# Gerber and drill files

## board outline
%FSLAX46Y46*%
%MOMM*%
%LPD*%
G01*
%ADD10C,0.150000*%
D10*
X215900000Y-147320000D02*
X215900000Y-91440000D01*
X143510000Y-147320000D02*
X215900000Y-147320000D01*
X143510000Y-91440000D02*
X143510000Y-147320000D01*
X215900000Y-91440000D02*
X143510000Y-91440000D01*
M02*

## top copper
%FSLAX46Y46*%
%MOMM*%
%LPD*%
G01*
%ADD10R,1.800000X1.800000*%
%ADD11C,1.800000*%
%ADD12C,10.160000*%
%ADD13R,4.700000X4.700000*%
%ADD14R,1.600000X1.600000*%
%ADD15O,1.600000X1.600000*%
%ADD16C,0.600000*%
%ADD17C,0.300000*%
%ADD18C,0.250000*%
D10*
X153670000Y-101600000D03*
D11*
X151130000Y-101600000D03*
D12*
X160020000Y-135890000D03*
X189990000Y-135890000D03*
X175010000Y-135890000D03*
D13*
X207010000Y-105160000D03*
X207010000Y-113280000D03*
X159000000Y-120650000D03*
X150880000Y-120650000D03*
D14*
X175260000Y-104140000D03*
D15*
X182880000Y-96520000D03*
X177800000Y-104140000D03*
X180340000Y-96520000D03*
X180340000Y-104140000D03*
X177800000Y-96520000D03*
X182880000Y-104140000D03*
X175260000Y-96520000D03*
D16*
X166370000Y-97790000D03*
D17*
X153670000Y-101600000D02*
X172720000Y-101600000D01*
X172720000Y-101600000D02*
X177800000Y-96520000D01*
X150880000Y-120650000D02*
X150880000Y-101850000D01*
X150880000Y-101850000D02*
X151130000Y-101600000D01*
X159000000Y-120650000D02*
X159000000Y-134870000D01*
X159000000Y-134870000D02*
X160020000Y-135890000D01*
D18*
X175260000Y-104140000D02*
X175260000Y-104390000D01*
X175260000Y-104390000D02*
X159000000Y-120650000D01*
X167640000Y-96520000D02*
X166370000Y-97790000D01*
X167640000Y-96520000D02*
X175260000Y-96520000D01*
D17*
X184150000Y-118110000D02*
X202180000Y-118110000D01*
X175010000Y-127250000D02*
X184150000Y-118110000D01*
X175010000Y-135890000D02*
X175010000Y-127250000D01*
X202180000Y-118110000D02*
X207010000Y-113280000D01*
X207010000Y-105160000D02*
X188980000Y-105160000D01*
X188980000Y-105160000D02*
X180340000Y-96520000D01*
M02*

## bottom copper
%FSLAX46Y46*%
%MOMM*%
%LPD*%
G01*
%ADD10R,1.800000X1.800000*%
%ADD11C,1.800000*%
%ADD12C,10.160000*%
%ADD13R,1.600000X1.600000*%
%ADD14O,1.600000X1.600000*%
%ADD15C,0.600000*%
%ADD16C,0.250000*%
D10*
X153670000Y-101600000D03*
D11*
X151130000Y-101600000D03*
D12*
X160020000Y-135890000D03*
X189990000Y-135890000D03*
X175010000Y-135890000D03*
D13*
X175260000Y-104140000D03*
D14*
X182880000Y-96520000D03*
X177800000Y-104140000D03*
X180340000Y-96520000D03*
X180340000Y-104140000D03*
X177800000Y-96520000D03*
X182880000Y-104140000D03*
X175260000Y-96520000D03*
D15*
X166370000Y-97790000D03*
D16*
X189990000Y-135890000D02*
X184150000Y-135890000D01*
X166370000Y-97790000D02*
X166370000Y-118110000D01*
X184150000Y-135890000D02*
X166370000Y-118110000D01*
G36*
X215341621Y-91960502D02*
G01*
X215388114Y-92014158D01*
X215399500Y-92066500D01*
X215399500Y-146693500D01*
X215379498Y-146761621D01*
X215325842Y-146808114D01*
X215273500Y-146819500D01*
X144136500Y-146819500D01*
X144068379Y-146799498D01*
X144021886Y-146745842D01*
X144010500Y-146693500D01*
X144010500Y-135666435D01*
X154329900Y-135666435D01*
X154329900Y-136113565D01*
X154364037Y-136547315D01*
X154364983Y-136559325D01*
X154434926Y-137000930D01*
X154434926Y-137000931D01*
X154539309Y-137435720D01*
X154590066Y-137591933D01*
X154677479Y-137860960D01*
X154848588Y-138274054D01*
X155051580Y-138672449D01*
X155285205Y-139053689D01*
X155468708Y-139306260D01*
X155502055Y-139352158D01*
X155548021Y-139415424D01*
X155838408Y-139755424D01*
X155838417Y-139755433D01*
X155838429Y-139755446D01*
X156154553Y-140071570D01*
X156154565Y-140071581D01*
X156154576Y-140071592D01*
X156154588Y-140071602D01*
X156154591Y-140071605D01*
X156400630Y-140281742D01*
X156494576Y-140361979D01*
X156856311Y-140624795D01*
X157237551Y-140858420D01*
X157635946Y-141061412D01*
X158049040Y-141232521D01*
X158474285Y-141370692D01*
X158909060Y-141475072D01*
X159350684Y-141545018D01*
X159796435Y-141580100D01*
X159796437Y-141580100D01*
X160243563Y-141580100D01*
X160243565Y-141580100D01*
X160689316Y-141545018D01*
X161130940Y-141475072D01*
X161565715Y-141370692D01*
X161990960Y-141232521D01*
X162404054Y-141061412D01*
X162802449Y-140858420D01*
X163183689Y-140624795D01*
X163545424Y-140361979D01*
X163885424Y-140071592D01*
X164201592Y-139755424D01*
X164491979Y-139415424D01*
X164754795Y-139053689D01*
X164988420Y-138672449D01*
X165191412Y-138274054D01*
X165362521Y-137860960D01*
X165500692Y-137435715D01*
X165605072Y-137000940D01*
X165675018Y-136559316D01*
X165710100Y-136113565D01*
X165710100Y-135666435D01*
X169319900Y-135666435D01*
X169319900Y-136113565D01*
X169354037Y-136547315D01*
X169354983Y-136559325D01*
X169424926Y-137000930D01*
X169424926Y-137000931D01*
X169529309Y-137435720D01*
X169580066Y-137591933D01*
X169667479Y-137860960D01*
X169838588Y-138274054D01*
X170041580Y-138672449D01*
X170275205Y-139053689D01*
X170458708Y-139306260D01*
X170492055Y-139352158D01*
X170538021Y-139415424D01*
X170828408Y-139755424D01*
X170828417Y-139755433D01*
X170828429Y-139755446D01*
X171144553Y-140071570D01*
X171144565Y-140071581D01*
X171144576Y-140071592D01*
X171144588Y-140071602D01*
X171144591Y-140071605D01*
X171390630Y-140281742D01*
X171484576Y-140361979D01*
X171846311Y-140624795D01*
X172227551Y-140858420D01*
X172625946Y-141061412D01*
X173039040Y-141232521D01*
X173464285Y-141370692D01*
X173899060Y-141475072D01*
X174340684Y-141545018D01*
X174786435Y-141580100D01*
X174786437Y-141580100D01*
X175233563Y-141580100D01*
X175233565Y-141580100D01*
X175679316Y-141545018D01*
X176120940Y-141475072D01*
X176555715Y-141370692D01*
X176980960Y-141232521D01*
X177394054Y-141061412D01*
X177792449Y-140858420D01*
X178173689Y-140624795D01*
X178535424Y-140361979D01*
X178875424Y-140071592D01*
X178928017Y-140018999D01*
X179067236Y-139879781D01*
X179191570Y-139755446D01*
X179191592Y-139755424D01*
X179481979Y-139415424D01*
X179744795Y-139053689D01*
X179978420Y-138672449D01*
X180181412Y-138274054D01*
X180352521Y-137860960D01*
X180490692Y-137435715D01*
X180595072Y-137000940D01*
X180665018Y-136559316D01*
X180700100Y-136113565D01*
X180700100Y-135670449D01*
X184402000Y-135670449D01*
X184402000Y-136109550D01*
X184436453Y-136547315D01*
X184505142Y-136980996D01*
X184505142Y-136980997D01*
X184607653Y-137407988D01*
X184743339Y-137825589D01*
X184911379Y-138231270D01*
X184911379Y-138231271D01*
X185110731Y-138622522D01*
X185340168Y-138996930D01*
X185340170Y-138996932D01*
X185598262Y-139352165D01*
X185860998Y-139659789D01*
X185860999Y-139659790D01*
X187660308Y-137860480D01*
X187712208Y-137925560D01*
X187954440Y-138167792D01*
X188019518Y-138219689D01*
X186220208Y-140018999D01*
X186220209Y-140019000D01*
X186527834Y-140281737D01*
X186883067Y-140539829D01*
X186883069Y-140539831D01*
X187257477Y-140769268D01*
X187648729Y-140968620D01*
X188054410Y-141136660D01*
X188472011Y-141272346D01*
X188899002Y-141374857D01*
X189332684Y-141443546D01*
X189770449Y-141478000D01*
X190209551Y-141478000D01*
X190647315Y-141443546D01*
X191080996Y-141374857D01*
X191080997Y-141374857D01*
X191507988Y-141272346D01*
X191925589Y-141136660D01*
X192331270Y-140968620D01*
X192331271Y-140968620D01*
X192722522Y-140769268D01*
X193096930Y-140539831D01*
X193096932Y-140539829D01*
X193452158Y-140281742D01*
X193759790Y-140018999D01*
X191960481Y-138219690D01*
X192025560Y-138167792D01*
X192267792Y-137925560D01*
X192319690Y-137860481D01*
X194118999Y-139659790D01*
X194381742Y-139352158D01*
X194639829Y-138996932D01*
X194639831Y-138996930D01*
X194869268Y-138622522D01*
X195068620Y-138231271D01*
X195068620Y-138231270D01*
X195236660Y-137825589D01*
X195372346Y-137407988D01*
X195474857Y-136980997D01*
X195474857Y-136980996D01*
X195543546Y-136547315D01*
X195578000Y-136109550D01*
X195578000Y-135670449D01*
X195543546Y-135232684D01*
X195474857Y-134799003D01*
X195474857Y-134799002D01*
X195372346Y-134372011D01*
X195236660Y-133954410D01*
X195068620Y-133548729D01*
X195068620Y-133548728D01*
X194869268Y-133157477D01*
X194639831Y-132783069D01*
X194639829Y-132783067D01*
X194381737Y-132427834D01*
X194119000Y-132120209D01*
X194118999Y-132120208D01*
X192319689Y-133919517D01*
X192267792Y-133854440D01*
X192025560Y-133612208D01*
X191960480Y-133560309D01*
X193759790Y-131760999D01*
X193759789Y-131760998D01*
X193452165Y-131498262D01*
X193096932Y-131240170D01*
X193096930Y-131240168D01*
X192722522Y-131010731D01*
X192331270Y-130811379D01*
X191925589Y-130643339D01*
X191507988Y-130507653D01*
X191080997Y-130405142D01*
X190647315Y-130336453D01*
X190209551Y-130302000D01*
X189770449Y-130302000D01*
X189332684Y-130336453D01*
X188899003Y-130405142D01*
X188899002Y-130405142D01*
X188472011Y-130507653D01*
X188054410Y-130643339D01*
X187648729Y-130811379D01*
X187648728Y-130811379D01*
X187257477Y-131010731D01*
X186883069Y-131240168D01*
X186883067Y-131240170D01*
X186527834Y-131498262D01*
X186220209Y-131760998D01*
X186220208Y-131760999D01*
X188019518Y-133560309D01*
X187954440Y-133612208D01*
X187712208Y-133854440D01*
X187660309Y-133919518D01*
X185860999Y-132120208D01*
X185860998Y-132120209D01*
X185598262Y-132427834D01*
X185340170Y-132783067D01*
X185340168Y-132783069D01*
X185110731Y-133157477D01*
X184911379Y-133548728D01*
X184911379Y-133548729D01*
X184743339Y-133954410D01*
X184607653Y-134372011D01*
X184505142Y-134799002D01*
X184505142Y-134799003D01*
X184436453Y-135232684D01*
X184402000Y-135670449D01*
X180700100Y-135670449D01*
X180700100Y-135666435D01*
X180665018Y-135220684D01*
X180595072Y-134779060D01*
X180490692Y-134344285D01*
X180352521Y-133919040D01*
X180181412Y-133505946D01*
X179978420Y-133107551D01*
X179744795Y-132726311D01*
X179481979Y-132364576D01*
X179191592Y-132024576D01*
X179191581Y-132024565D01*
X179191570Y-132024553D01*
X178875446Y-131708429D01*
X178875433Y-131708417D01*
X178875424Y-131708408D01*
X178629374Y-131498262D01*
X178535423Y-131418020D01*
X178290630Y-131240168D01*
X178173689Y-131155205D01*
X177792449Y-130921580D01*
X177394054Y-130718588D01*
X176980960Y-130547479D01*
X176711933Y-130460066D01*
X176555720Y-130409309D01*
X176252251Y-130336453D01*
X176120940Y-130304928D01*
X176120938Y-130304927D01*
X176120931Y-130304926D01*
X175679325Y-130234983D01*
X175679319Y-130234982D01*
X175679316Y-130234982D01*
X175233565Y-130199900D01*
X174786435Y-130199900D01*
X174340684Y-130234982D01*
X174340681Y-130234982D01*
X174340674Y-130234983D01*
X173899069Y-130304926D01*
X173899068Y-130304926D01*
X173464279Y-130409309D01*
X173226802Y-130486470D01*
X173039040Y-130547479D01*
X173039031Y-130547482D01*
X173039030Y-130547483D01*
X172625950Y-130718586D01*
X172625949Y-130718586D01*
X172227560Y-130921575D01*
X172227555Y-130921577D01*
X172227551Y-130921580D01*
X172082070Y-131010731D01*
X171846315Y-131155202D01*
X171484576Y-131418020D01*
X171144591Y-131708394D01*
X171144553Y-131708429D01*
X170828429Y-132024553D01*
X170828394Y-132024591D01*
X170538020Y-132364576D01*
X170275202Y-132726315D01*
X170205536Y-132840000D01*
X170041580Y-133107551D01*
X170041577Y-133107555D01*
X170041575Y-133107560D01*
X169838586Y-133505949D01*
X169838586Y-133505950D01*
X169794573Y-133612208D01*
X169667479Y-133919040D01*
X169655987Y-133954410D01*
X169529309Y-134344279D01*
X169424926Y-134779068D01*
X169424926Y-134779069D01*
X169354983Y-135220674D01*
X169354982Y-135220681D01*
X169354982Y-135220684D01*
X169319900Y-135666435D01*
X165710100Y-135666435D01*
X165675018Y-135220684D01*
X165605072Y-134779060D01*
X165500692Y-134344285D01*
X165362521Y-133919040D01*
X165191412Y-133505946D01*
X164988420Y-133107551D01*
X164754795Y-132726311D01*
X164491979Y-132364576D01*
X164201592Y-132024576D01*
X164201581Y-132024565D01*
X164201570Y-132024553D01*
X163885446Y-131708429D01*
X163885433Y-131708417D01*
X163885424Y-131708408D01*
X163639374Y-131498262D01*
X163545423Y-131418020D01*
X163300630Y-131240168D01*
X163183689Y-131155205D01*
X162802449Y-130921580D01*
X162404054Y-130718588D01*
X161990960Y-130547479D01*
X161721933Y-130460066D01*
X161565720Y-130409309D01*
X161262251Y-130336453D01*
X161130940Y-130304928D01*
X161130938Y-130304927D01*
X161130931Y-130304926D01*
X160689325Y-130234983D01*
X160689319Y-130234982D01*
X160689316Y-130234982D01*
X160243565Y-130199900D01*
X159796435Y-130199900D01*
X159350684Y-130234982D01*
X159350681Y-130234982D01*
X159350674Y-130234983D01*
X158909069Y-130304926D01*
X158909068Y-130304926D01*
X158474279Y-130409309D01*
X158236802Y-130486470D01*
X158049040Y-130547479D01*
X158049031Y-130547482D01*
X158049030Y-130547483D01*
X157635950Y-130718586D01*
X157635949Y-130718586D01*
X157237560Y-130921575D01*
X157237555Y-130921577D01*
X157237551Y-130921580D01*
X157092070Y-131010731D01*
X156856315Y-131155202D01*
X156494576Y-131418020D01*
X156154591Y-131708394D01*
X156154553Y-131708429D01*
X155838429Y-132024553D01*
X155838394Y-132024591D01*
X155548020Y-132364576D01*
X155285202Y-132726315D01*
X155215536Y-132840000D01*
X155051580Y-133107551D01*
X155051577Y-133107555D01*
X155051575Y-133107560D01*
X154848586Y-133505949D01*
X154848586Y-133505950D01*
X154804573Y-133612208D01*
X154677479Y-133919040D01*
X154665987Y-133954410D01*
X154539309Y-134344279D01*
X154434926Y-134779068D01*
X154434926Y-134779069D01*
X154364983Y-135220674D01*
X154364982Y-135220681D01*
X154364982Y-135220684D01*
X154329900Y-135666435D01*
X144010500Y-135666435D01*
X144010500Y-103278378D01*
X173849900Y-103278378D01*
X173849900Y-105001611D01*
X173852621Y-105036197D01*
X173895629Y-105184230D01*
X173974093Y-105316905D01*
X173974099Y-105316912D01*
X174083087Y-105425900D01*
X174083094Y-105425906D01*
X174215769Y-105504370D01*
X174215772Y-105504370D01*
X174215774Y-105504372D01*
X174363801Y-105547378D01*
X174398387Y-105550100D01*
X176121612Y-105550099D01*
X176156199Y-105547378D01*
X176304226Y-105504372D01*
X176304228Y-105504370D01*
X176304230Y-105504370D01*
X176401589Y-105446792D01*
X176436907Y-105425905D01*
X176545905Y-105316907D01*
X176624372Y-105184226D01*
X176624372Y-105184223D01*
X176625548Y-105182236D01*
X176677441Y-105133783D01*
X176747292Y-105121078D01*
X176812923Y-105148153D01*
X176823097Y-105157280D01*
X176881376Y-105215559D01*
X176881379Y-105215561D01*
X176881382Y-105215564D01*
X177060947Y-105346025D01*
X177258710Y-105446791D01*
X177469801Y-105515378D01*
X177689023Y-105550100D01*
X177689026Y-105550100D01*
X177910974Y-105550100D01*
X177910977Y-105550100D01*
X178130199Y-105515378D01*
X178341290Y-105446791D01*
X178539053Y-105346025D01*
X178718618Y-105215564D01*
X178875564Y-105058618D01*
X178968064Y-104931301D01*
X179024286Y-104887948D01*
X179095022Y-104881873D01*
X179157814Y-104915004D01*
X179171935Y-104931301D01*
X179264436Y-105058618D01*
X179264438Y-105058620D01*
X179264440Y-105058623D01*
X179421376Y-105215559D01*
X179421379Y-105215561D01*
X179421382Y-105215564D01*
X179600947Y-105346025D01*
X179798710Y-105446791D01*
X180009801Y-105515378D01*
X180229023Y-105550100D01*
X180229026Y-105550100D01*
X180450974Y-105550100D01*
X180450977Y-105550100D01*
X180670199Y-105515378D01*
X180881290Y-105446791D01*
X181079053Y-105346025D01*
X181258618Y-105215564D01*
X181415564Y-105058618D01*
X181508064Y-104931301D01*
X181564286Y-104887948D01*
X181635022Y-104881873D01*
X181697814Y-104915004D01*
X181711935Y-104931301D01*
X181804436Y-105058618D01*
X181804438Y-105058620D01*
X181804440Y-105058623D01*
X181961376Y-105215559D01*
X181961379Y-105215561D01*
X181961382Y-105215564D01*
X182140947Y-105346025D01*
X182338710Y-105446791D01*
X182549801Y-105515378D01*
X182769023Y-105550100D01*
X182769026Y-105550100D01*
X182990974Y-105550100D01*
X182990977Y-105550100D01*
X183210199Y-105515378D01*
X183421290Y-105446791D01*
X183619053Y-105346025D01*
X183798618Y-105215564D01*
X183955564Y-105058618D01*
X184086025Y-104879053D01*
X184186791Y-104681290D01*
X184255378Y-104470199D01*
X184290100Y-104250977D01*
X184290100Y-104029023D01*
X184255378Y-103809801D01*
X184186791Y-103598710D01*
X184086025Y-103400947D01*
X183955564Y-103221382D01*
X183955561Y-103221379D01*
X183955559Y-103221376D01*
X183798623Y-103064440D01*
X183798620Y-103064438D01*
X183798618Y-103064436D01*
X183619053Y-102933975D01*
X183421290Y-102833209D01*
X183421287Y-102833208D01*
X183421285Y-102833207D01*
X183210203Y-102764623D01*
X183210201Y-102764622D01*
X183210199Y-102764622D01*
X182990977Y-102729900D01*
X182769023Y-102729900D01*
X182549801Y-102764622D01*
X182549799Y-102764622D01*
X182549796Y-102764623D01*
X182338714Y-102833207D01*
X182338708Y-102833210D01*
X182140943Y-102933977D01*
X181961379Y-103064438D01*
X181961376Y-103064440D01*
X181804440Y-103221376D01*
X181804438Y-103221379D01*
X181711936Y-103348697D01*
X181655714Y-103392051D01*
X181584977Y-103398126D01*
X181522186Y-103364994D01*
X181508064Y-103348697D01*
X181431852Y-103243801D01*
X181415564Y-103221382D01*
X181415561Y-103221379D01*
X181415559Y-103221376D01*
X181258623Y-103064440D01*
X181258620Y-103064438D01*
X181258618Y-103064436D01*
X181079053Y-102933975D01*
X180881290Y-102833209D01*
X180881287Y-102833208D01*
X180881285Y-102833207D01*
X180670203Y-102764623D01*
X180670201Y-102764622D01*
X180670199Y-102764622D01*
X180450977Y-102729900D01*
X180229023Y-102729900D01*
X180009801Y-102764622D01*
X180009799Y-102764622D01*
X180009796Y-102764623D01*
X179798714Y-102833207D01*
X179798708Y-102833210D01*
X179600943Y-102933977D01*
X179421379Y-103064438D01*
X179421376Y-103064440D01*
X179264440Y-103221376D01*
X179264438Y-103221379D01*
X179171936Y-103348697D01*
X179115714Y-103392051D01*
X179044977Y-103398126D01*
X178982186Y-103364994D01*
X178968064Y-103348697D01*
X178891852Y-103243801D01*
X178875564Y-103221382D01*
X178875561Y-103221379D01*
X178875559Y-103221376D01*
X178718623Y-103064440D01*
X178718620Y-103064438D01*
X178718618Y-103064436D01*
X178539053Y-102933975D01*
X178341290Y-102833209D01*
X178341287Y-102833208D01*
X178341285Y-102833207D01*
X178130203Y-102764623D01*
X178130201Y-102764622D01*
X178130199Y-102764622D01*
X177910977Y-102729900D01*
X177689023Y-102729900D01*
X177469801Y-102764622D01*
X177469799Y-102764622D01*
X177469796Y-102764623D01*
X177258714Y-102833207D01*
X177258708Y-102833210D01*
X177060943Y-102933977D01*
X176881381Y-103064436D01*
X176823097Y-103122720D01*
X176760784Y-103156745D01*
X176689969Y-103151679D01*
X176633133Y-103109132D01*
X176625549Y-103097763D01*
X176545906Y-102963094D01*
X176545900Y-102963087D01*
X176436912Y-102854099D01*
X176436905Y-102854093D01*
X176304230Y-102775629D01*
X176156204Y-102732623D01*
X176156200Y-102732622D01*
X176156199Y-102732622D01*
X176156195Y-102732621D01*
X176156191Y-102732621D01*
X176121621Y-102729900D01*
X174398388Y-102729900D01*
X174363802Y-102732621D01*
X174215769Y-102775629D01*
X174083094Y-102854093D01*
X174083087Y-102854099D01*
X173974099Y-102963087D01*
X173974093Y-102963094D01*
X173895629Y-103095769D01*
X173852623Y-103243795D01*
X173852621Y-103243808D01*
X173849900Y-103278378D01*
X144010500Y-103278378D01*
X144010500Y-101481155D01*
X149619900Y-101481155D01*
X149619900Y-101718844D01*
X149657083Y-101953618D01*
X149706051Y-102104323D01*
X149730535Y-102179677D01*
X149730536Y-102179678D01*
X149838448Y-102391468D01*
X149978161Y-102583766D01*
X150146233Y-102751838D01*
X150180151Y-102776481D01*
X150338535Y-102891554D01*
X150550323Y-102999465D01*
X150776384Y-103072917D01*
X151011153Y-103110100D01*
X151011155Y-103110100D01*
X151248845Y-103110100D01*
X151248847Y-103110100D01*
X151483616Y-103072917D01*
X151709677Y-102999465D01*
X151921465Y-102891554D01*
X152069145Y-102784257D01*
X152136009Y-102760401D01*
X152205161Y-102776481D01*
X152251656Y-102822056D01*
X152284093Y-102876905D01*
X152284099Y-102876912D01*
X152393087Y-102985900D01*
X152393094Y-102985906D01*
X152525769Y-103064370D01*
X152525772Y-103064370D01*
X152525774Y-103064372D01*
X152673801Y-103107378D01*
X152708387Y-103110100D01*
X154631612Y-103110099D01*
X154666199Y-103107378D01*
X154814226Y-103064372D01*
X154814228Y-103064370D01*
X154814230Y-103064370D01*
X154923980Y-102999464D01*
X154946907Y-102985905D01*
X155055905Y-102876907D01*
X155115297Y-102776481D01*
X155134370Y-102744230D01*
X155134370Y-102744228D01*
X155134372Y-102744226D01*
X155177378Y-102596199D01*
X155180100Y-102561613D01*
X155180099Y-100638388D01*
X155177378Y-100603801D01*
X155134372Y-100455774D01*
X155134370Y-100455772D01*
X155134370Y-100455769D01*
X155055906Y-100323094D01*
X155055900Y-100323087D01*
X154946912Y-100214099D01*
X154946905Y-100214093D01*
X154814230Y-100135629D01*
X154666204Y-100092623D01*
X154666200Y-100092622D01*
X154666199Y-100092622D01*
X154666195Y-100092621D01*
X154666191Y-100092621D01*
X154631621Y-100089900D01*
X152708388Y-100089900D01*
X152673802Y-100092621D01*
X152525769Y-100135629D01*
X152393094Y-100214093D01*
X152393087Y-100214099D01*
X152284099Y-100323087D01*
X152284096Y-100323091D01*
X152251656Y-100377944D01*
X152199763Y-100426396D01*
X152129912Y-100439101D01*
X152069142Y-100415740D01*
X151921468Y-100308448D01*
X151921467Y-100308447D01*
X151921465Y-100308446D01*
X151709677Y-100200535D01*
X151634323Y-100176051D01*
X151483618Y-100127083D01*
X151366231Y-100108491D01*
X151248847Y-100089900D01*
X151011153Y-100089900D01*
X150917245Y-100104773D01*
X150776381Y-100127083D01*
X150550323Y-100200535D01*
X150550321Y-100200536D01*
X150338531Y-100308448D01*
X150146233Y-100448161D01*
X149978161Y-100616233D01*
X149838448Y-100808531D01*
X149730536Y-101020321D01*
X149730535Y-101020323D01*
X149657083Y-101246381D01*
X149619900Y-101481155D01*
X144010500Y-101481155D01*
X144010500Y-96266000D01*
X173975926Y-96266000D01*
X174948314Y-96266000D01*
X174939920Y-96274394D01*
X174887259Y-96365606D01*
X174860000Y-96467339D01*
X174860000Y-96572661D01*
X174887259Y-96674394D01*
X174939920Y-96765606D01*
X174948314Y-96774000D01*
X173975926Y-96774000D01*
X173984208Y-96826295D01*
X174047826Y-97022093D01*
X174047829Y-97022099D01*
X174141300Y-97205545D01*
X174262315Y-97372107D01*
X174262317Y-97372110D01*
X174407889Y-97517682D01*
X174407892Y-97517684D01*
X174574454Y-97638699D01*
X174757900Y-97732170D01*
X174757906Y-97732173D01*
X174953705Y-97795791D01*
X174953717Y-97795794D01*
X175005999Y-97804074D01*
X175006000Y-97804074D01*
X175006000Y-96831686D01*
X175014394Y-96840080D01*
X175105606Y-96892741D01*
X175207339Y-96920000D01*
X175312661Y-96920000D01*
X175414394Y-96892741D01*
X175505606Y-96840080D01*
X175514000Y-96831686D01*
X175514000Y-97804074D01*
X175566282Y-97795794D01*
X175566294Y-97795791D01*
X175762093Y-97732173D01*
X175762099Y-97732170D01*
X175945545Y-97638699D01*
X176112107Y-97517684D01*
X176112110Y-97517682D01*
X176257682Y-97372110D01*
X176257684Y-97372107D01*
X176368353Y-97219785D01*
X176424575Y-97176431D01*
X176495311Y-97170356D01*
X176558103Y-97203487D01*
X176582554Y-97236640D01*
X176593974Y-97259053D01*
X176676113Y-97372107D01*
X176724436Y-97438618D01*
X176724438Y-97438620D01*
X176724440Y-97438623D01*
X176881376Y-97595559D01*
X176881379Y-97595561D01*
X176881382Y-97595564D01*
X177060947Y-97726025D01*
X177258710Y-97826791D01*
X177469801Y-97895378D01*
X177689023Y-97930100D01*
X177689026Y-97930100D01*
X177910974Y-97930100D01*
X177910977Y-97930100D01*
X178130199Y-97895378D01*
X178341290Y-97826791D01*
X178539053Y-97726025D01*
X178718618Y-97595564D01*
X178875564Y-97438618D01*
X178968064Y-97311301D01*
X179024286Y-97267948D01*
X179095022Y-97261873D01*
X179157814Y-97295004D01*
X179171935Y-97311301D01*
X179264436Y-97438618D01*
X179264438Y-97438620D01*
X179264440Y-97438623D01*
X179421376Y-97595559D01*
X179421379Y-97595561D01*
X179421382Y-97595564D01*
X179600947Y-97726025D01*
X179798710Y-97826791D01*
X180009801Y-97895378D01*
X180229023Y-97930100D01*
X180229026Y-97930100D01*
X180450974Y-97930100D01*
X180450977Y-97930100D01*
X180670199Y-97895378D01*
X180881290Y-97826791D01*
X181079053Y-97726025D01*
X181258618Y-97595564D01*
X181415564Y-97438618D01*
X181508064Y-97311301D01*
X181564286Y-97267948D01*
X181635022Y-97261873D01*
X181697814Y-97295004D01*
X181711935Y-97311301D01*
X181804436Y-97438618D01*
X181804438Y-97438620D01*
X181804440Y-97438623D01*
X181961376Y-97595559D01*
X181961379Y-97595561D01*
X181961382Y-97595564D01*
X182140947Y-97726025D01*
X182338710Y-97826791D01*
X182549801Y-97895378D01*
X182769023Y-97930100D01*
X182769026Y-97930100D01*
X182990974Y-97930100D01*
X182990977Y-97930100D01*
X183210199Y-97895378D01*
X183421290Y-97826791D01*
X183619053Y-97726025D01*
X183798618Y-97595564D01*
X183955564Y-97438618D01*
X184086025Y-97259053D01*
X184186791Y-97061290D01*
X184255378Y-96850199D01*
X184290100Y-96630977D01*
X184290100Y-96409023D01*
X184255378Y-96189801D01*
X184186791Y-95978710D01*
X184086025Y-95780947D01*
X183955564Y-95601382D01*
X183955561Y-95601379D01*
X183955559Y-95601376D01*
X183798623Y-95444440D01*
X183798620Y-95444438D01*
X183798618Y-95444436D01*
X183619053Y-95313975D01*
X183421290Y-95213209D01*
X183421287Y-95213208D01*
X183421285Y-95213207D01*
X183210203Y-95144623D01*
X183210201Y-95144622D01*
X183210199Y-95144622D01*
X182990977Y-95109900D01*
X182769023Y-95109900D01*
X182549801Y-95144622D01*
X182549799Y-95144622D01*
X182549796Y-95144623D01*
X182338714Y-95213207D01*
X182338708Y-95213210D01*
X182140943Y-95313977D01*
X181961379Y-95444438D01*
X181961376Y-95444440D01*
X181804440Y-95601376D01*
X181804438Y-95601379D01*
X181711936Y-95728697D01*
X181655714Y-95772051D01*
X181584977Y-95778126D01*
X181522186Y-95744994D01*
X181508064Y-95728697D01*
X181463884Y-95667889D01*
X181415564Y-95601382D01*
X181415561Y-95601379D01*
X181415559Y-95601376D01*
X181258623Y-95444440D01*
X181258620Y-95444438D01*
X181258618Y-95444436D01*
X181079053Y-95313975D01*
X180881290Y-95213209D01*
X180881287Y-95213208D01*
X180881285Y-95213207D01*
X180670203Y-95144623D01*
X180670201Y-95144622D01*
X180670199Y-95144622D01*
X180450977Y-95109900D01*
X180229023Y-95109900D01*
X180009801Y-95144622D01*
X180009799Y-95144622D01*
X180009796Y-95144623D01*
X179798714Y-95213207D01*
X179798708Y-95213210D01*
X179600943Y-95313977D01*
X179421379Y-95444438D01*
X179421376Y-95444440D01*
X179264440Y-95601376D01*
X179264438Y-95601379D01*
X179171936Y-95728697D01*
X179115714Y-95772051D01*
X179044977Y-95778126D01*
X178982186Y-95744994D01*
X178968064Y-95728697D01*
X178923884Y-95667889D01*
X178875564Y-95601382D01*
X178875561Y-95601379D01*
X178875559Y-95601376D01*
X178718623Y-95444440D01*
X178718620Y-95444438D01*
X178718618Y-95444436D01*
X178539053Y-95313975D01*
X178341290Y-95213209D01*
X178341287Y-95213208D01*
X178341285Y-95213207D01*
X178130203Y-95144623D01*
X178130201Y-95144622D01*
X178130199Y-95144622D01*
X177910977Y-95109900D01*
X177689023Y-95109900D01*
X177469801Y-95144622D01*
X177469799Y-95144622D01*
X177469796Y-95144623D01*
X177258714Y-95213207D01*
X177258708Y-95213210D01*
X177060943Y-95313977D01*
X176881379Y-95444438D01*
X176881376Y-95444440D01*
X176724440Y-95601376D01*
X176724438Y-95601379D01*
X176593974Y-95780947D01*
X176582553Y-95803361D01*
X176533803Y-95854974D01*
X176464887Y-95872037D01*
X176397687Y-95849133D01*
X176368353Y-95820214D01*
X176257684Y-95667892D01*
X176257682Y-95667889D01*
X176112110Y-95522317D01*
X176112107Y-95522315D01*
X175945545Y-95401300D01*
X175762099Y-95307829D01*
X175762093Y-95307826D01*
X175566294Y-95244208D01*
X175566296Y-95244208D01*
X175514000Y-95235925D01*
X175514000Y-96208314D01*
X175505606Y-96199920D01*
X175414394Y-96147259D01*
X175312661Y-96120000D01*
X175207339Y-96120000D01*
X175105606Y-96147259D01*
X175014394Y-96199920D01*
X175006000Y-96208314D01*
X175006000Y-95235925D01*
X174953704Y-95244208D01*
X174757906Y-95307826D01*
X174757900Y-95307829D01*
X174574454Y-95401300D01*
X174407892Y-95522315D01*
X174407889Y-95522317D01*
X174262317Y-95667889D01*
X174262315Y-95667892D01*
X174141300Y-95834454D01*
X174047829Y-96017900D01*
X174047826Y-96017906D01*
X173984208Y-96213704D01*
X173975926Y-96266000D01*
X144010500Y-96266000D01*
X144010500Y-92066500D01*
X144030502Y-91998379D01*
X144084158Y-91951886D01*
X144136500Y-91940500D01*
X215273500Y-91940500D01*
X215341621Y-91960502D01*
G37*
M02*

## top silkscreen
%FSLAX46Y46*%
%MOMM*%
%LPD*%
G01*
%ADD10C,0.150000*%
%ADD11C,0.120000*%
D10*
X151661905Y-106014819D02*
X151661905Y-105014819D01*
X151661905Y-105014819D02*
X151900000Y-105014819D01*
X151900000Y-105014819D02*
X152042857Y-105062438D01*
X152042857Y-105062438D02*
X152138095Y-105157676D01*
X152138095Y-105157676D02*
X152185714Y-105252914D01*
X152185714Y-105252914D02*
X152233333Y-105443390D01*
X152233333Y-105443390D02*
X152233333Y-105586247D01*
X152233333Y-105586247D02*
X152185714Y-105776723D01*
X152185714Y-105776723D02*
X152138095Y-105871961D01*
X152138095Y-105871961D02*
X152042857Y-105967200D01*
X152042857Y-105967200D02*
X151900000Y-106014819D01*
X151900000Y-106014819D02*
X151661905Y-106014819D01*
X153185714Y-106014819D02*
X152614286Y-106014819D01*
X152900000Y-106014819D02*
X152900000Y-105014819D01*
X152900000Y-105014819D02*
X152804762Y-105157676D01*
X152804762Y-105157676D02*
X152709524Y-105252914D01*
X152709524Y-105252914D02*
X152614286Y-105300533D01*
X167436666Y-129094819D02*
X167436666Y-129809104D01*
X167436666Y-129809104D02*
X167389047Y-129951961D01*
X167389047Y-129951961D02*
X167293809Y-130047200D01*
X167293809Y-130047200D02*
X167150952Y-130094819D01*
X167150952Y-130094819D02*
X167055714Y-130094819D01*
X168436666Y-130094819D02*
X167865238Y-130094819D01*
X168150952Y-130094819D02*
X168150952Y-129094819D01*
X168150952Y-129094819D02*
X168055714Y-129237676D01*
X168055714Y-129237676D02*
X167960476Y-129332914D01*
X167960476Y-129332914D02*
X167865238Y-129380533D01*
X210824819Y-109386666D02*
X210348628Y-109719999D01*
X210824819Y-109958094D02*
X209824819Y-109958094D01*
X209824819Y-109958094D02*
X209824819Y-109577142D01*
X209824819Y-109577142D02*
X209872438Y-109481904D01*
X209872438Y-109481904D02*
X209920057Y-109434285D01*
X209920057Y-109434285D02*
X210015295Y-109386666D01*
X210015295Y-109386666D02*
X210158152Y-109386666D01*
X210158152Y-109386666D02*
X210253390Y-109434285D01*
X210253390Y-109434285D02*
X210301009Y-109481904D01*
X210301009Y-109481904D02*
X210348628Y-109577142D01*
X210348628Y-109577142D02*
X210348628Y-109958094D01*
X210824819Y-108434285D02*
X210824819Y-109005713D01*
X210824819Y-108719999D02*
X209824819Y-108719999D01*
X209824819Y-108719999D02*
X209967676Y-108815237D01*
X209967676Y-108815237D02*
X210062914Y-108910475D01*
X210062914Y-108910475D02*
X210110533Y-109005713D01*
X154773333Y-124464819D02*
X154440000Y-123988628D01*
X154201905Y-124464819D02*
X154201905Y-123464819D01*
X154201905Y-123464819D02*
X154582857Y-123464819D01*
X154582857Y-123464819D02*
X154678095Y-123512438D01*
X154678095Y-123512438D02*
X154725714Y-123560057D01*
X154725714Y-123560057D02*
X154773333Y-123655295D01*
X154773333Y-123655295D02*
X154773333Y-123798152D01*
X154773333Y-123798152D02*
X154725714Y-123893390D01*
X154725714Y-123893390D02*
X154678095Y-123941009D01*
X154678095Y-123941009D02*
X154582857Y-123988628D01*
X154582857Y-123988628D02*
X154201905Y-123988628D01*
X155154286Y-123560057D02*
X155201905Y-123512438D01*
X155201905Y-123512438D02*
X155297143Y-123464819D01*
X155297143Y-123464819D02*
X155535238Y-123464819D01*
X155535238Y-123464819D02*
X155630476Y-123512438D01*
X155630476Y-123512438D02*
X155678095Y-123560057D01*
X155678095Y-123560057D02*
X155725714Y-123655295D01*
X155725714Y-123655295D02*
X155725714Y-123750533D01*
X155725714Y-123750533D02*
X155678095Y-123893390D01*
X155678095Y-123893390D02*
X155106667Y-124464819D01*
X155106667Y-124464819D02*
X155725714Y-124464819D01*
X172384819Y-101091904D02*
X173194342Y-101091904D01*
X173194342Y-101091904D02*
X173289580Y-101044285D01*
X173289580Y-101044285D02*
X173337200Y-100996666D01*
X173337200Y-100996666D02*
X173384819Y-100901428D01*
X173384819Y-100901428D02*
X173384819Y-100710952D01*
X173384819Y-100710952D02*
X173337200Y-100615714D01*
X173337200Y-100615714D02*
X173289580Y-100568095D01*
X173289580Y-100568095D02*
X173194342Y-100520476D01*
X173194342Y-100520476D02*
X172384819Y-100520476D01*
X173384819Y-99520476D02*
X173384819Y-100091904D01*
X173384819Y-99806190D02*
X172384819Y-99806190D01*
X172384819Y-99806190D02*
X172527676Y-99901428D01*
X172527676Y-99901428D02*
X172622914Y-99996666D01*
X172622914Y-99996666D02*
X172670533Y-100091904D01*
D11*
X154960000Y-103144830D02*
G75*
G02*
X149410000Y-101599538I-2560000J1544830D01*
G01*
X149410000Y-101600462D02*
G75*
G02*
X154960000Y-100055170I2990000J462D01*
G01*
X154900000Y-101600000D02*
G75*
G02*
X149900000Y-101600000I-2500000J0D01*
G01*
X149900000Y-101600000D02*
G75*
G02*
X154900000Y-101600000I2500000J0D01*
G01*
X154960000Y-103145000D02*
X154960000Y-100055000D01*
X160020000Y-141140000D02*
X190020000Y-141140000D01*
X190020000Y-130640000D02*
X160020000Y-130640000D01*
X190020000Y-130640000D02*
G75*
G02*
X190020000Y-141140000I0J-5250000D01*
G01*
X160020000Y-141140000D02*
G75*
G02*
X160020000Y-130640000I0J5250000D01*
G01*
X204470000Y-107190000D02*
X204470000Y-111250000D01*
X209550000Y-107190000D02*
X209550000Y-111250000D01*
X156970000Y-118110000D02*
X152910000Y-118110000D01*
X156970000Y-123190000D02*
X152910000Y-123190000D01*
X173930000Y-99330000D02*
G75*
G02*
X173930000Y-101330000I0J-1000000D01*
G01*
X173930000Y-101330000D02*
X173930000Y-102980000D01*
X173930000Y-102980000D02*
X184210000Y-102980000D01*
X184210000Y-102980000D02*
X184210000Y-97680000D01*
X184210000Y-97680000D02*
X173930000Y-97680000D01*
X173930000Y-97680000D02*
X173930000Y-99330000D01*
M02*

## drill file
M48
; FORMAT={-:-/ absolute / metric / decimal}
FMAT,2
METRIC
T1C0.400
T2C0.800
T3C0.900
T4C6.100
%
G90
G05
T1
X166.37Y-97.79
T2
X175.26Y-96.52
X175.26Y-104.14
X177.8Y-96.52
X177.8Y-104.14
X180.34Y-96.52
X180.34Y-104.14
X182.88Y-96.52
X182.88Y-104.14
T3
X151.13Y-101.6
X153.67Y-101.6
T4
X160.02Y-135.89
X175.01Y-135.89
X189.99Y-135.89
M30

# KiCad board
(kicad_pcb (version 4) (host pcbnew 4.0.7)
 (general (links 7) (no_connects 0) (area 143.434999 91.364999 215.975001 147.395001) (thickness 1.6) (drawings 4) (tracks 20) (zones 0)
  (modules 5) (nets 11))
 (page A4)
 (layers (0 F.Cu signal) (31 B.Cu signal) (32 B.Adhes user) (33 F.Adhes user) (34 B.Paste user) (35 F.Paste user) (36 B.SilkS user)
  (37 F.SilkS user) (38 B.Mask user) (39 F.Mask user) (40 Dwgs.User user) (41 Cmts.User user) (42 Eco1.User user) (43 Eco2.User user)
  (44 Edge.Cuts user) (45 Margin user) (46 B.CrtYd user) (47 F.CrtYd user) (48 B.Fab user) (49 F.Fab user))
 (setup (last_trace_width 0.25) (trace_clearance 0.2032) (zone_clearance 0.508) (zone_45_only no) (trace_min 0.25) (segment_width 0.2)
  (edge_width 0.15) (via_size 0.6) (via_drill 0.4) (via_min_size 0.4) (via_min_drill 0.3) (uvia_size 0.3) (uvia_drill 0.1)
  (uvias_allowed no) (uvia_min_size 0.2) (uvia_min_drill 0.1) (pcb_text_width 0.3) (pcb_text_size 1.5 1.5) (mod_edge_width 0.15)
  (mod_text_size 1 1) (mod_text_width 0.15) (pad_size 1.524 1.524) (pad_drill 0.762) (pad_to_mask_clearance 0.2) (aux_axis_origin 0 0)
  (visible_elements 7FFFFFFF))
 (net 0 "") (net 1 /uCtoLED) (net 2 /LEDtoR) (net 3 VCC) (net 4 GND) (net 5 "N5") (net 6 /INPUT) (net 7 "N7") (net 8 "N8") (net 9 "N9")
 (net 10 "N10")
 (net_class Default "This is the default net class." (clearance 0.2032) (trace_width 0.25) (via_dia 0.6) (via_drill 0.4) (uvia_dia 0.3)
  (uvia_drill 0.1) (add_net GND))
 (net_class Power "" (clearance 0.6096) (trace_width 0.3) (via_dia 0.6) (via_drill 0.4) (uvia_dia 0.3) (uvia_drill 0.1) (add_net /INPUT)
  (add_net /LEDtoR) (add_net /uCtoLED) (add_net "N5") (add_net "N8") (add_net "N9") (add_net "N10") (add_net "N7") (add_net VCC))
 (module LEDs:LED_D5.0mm (layer F.Cu) (at 153.67 101.6 180)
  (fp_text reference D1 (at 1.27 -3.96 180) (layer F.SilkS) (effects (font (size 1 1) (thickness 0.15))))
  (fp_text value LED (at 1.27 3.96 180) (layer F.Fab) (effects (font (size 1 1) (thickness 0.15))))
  (fp_arc (start 1.27 0) (end -1.29 -1.54483) (angle 148.9) (layer F.SilkS) (width 0.12))
  (fp_arc (start 1.27 0) (end -1.29 1.54483) (angle -148.9) (layer F.SilkS) (width 0.12))
  (fp_circle (center 1.27 0) (end 3.77 0) (layer F.SilkS) (width 0.12))
  (fp_line (start -1.29 -1.545) (end -1.29 1.545) (layer F.SilkS) (width 0.12))
  (pad 1 thru_hole rect (at 0 0 180) (size 1.8 1.8) (drill 0.9) (layers *.Cu *.Mask) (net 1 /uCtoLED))
  (pad 2 thru_hole circle (at 2.54 0 180) (size 1.8 1.8) (drill 0.9) (layers *.Cu *.Mask) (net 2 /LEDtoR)))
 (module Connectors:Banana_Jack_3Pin (layer F.Cu) (at 160.02 135.89)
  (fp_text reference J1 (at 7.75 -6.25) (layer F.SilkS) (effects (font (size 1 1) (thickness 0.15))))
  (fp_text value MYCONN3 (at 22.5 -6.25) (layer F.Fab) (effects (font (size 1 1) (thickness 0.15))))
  (fp_line (start 0 5.25) (end 30 5.25) (layer F.SilkS) (width 0.12))
  (fp_line (start 30 -5.25) (end 0 -5.25) (layer F.SilkS) (width 0.12))
  (fp_arc (start 30 0) (end 30 -5.25) (angle 180) (layer F.SilkS) (width 0.12))
  (fp_arc (start 0 0) (end 0 5.25) (angle 180) (layer F.SilkS) (width 0.12))
  (pad 1 thru_hole circle (at 0 0) (size 10.16 10.16) (drill 6.1) (layers *.Cu *.Mask) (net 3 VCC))
  (pad 3 thru_hole circle (at 29.97 0) (size 10.16 10.16) (drill 6.1) (layers *.Cu *.Mask) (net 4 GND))
  (pad 2 thru_hole circle (at 14.99 0) (size 10.16 10.16) (drill 6.1) (layers *.Cu *.Mask) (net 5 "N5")))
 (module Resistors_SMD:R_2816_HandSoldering (layer F.Cu) (at 207.01 109.22 270)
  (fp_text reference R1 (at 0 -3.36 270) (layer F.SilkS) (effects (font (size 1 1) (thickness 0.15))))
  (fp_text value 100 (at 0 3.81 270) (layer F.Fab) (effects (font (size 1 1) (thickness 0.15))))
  (fp_line (start -2.03 2.54) (end 2.03 2.54) (layer F.SilkS) (width 0.12))
  (fp_line (start -2.03 -2.54) (end 2.03 -2.54) (layer F.SilkS) (width 0.12))
  (pad 1 smd rect (at -4.06 0 270) (size 4.7 4.7) (layers F.Cu F.Paste F.Mask) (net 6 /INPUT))
  (pad 2 smd rect (at 4.06 0 270) (size 4.7 4.7) (layers F.Cu F.Paste F.Mask) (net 5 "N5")))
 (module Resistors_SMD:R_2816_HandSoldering (layer F.Cu) (at 154.94 120.65 180)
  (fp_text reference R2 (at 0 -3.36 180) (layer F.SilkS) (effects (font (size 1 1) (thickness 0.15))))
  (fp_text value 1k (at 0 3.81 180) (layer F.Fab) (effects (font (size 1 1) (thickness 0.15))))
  (fp_line (start -2.03 2.54) (end 2.03 2.54) (layer F.SilkS) (width 0.12))
  (fp_line (start -2.03 -2.54) (end 2.03 -2.54) (layer F.SilkS) (width 0.12))
  (pad 1 smd rect (at -4.06 0 180) (size 4.7 4.7) (layers F.Cu F.Paste F.Mask) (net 3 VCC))
  (pad 2 smd rect (at 4.06 0 180) (size 4.7 4.7) (layers F.Cu F.Paste F.Mask) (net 2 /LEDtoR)))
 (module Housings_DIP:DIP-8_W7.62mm (layer F.Cu) (at 175.26 104.14 90)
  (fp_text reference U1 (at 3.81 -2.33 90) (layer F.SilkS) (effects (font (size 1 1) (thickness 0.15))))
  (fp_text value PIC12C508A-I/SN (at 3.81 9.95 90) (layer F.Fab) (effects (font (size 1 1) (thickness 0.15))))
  (fp_arc (start 3.81 -1.33) (end 2.81 -1.33) (angle -180) (layer F.SilkS) (width 0.12))
  (fp_line (start 2.81 -1.33) (end 1.16 -1.33) (layer F.SilkS) (width 0.12))
  (fp_line (start 1.16 -1.33) (end 1.16 8.95) (layer F.SilkS) (width 0.12))
  (fp_line (start 1.16 8.95) (end 6.46 8.95) (layer F.SilkS) (width 0.12))
  (fp_line (start 6.46 8.95) (end 6.46 -1.33) (layer F.SilkS) (width 0.12))
  (fp_line (start 6.46 -1.33) (end 4.81 -1.33) (layer F.SilkS) (width 0.12))
  (pad 1 thru_hole rect (at 0 0 90) (size 1.6 1.6) (drill 0.8) (layers *.Cu *.Mask) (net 3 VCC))
  (pad 5 thru_hole oval (at 7.62 7.62 90) (size 1.6 1.6) (drill 0.8) (layers *.Cu *.Mask) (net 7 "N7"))
  (pad 2 thru_hole oval (at 0 2.54 90) (size 1.6 1.6) (drill 0.8) (layers *.Cu *.Mask) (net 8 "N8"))
  (pad 6 thru_hole oval (at 7.62 5.08 90) (size 1.6 1.6) (drill 0.8) (layers *.Cu *.Mask) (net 6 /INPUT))
  (pad 3 thru_hole oval (at 0 5.08 90) (size 1.6 1.6) (drill 0.8) (layers *.Cu *.Mask) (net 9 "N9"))
  (pad 7 thru_hole oval (at 7.62 2.54 90) (size 1.6 1.6) (drill 0.8) (layers *.Cu *.Mask) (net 1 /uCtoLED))
  (pad 4 thru_hole oval (at 0 7.62 90) (size 1.6 1.6) (drill 0.8) (layers *.Cu *.Mask) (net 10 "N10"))
  (pad 8 thru_hole oval (at 7.62 0 90) (size 1.6 1.6) (drill 0.8) (layers *.Cu *.Mask) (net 4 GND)))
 (gr_line (start 215.9 147.32) (end 215.9 91.44) (angle 90) (layer Edge.Cuts) (width 0.15))
 (gr_line (start 143.51 147.32) (end 215.9 147.32) (angle 90) (layer Edge.Cuts) (width 0.15))
 (gr_line (start 143.51 91.44) (end 143.51 147.32) (angle 90) (layer Edge.Cuts) (width 0.15))
 (gr_line (start 215.9 91.44) (end 143.51 91.44) (angle 90) (layer Edge.Cuts) (width 0.15))
 (segment (start 153.67 101.6) (end 172.72 101.6) (width 0.3) (layer F.Cu) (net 1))
 (segment (start 172.72 101.6) (end 177.8 96.52) (width 0.3) (layer F.Cu) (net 1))
 (segment (start 150.88 120.65) (end 150.88 101.85) (width 0.3) (layer F.Cu) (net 2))
 (segment (start 150.88 101.85) (end 151.13 101.6) (width 0.3) (layer F.Cu) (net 2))
 (segment (start 159 120.65) (end 159 134.87) (width 0.3) (layer F.Cu) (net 3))
 (segment (start 159 134.87) (end 160.02 135.89) (width 0.3) (layer F.Cu) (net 3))
 (segment (start 175.26 104.14) (end 175.26 104.39) (width 0.25) (layer F.Cu) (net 3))
 (segment (start 175.26 104.39) (end 159 120.65) (width 0.25) (layer F.Cu) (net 3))
 (segment (start 189.99 135.89) (end 184.15 135.89) (width 0.25) (layer B.Cu) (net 4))
 (segment (start 167.64 96.52) (end 166.37 97.79) (width 0.25) (layer F.Cu) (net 4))
 (via (at 166.37 97.79) (size 0.6) (drill 0.4) (layers F.Cu B.Cu) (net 4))
 (segment (start 166.37 97.79) (end 166.37 118.11) (width 0.25) (layer B.Cu) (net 4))
 (segment (start 167.64 96.52) (end 175.26 96.52) (width 0.25) (layer F.Cu) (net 4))
 (segment (start 184.15 135.89) (end 166.37 118.11) (width 0.25) (layer B.Cu) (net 4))
 (segment (start 184.15 118.11) (end 202.18 118.11) (width 0.3) (layer F.Cu) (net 5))
 (segment (start 175.01 127.25) (end 184.15 118.11) (width 0.3) (layer F.Cu) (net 5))
 (segment (start 175.01 135.89) (end 175.01 127.25) (width 0.3) (layer F.Cu) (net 5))
 (segment (start 202.18 118.11) (end 207.01 113.28) (width 0.3) (layer F.Cu) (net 5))
 (segment (start 207.01 105.16) (end 188.98 105.16) (width 0.3) (layer F.Cu) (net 6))
 (segment (start 188.98 105.16) (end 180.34 96.52) (width 0.3) (layer F.Cu) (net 6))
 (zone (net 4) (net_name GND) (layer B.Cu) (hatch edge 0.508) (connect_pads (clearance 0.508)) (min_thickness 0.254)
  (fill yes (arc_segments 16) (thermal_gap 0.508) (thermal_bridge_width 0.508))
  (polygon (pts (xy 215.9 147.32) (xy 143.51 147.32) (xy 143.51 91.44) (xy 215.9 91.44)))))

